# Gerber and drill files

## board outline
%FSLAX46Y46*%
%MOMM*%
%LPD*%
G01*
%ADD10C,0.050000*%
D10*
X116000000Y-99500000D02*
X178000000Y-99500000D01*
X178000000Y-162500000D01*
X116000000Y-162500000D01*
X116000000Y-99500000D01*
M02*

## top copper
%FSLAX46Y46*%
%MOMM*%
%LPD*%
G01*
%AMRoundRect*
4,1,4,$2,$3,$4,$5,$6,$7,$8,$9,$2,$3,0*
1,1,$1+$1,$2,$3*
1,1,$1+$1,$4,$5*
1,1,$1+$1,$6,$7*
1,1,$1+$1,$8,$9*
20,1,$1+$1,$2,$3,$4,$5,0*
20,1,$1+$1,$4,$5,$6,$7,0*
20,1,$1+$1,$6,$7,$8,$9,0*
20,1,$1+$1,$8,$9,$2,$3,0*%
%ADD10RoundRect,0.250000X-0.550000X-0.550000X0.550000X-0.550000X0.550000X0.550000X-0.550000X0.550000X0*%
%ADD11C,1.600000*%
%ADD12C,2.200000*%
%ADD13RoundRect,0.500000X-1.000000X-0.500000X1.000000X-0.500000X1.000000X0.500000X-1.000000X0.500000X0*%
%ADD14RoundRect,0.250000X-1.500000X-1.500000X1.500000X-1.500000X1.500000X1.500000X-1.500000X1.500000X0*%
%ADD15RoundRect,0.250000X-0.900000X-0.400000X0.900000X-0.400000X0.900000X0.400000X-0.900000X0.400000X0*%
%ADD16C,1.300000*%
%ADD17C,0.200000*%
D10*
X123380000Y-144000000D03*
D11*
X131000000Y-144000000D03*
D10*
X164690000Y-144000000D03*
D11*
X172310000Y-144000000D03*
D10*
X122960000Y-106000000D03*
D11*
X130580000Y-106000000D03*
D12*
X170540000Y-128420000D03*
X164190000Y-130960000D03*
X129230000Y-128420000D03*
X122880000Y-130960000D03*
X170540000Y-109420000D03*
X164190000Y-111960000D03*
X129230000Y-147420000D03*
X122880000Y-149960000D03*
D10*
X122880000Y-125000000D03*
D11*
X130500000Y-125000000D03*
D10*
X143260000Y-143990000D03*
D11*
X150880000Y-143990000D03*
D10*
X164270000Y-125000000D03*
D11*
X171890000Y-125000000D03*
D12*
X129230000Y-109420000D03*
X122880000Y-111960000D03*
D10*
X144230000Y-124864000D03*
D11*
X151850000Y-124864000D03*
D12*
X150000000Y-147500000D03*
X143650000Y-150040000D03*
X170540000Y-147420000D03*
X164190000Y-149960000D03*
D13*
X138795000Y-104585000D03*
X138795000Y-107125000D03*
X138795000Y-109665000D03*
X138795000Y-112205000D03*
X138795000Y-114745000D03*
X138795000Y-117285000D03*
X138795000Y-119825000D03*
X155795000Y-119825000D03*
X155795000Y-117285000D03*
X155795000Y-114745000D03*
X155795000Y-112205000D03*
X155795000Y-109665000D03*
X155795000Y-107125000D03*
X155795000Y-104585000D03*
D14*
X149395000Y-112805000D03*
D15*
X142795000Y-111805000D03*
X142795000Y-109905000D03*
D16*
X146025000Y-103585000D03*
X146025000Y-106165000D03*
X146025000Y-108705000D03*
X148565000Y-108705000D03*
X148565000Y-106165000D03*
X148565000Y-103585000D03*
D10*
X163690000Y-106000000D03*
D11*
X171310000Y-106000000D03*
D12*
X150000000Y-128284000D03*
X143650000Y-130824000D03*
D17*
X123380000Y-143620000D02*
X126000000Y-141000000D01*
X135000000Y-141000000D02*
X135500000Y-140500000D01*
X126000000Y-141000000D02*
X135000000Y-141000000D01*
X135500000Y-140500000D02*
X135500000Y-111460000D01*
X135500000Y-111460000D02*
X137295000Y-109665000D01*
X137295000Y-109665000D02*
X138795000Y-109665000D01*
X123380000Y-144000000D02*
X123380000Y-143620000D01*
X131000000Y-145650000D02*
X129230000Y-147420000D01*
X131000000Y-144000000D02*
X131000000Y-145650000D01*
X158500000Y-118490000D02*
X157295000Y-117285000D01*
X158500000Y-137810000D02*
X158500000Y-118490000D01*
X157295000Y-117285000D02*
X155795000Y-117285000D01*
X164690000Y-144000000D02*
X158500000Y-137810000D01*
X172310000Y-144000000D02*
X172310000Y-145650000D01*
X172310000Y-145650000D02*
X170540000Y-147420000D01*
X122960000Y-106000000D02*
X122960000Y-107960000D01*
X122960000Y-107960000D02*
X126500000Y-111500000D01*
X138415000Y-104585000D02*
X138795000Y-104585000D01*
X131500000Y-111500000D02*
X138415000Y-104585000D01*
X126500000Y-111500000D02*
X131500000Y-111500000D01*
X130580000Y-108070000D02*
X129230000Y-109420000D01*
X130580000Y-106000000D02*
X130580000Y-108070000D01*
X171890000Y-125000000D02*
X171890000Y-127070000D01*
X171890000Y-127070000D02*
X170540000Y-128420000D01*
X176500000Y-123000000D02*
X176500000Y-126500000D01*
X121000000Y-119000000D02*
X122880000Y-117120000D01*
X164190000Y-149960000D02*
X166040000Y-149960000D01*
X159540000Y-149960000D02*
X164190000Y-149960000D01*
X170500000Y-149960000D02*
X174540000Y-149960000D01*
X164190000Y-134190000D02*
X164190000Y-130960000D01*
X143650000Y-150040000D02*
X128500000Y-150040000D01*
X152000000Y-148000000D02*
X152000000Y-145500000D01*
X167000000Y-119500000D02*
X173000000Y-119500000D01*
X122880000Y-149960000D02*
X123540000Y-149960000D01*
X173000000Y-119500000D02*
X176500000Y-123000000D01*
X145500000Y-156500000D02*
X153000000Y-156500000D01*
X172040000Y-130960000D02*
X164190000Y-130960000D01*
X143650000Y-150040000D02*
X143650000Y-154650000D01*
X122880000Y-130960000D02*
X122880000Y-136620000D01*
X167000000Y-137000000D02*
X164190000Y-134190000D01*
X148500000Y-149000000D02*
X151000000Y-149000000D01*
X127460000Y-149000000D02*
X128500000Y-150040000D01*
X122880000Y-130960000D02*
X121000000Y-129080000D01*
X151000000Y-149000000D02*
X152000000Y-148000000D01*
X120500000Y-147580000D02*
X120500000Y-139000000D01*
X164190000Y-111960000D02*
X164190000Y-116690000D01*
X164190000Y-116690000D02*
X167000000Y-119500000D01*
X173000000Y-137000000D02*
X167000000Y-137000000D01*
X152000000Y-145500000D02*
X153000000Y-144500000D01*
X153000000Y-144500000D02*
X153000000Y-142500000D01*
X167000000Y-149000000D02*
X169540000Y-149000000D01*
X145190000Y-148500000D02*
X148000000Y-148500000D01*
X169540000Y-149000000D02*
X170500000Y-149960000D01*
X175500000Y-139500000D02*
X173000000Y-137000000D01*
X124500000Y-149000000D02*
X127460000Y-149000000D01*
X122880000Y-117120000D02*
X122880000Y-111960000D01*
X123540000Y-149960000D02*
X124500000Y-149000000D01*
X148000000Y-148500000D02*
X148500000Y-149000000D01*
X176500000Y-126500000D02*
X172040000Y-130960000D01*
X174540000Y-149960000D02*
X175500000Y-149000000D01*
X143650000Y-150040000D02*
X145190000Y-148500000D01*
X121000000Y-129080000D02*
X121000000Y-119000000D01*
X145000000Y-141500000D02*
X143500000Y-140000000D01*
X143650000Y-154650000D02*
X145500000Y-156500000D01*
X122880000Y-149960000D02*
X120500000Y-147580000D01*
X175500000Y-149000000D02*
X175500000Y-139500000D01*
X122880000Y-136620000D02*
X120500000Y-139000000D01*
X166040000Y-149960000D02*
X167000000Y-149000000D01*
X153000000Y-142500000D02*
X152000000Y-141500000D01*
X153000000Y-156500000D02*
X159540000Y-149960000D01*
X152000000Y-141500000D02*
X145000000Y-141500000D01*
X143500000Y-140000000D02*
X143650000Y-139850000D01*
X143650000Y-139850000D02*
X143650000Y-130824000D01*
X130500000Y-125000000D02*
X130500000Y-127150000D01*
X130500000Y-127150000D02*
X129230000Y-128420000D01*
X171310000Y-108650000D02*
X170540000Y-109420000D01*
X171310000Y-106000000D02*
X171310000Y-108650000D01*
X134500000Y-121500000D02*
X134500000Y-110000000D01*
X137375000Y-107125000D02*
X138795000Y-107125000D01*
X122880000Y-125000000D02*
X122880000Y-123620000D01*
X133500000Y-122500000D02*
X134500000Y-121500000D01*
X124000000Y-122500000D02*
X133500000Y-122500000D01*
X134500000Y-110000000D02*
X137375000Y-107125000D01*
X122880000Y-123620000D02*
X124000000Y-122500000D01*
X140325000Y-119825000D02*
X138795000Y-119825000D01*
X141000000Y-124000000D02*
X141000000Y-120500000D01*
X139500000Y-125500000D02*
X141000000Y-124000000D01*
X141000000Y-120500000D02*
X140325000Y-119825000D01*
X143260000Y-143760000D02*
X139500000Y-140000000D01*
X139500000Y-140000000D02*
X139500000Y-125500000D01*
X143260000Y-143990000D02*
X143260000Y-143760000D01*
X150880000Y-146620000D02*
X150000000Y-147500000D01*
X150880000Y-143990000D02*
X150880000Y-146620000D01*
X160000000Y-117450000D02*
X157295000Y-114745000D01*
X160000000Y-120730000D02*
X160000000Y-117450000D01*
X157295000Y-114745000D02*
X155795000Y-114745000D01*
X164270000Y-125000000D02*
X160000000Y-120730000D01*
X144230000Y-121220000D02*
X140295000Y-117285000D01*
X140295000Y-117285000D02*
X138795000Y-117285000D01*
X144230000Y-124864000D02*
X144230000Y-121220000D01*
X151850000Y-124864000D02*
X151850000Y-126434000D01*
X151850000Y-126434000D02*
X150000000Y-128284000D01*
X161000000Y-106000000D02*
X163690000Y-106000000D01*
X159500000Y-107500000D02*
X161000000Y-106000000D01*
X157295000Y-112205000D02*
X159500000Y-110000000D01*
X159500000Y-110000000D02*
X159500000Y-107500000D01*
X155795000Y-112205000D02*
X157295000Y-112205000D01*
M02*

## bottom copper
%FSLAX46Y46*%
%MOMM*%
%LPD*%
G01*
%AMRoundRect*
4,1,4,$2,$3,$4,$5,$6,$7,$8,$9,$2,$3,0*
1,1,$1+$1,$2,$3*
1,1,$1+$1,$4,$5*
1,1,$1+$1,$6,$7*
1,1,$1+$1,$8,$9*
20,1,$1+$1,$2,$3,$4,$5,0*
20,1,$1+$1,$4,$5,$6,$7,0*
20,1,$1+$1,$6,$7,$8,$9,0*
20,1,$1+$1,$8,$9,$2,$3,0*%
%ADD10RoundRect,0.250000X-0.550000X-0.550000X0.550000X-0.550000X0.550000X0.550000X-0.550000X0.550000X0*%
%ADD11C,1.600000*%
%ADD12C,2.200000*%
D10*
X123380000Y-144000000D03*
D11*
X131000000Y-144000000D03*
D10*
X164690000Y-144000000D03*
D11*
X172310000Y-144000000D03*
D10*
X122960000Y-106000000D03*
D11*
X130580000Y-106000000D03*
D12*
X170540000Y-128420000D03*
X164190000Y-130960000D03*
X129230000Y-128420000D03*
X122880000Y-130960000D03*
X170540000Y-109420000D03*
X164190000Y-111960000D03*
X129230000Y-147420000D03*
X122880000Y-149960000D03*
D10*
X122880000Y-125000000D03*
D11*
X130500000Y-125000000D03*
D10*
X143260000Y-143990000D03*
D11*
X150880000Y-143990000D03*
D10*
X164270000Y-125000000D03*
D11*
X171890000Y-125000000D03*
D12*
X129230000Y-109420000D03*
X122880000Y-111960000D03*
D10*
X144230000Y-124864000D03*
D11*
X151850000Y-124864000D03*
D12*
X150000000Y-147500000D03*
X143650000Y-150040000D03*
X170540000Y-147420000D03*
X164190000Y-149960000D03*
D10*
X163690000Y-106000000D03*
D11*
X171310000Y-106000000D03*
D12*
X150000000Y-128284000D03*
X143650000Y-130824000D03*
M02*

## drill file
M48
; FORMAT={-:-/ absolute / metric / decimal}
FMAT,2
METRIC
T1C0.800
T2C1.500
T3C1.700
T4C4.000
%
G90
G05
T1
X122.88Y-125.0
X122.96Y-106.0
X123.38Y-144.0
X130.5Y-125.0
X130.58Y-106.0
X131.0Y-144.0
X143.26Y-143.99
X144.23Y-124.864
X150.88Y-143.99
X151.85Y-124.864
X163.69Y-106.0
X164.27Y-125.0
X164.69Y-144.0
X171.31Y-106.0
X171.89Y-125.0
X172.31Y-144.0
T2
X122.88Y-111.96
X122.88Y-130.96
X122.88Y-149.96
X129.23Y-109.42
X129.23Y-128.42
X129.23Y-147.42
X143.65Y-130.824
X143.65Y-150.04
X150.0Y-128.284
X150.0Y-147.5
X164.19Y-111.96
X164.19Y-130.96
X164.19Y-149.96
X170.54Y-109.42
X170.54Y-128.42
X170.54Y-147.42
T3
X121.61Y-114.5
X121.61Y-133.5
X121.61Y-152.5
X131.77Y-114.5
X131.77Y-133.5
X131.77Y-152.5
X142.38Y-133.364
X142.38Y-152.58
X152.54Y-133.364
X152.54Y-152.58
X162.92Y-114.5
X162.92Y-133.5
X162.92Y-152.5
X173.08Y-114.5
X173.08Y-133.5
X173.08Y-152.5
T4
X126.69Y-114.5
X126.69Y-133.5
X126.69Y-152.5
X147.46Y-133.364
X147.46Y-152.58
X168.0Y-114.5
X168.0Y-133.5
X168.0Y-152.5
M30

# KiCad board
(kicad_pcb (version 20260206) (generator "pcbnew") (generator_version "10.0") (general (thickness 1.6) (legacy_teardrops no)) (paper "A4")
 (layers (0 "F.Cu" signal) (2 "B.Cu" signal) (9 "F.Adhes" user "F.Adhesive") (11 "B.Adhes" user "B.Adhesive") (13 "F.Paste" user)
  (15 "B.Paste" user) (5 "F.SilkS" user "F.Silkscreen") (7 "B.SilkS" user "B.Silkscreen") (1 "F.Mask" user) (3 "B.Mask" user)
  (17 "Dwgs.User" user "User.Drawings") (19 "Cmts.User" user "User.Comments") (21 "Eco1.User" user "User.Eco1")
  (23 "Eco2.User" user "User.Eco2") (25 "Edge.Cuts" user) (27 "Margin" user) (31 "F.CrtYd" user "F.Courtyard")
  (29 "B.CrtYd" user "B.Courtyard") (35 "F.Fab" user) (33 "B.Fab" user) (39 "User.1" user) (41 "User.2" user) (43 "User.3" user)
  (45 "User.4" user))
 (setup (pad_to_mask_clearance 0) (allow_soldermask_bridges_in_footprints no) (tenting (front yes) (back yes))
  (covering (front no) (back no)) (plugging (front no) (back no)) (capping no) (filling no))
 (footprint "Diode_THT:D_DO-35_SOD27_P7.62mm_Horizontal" (layer "F.Cu") (at 123.38 144)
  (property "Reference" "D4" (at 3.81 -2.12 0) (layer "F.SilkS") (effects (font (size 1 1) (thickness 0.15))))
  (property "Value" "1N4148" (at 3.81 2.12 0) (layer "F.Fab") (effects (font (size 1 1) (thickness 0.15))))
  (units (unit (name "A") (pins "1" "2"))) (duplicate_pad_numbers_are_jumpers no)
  (pad "1" thru_hole roundrect (at 0 0) (size 1.6 1.6) (drill 0.8) (layers "*.Cu" "*.Mask") (remove_unused_layers no)
   (roundrect_rratio 0.15625) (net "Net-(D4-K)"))
  (pad "2" thru_hole circle (at 7.62 0) (size 1.6 1.6) (drill 0.8) (layers "*.Cu" "*.Mask") (remove_unused_layers no) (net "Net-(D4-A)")))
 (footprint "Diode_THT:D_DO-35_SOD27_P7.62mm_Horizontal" (layer "F.Cu") (at 164.69 144)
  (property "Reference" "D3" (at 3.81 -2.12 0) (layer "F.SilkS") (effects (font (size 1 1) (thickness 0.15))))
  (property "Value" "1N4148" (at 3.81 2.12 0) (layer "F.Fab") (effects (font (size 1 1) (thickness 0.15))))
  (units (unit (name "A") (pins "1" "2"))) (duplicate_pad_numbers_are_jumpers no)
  (pad "1" thru_hole roundrect (at 0 0) (size 1.6 1.6) (drill 0.8) (layers "*.Cu" "*.Mask") (remove_unused_layers no)
   (roundrect_rratio 0.15625) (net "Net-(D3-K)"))
  (pad "2" thru_hole circle (at 7.62 0) (size 1.6 1.6) (drill 0.8) (layers "*.Cu" "*.Mask") (remove_unused_layers no) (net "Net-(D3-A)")))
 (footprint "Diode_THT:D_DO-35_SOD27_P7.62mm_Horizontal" (layer "F.Cu") (at 122.96 106)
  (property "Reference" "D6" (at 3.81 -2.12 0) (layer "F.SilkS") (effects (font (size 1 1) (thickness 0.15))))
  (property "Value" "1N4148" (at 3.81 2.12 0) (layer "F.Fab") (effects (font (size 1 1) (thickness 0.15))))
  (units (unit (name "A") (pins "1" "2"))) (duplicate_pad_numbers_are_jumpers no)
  (pad "1" thru_hole roundrect (at 0 0) (size 1.6 1.6) (drill 0.8) (layers "*.Cu" "*.Mask") (remove_unused_layers no)
   (roundrect_rratio 0.15625) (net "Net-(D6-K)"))
  (pad "2" thru_hole circle (at 7.62 0) (size 1.6 1.6) (drill 0.8) (layers "*.Cu" "*.Mask") (remove_unused_layers no) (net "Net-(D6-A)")))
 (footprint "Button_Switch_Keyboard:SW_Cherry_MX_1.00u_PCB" (layer "F.Cu") (at 170.54 128.42)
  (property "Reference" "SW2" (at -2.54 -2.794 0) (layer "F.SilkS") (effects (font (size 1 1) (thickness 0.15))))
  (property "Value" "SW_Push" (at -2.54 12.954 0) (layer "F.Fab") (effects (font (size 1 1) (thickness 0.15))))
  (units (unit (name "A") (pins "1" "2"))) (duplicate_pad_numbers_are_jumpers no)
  (pad "" np_thru_hole circle (at -7.62 5.08) (size 1.7 1.7) (drill 1.7) (layers "*.Cu" "*.Mask"))
  (pad "" np_thru_hole circle (at -2.54 5.08) (size 4 4) (drill 4) (layers "*.Cu" "*.Mask"))
  (pad "" np_thru_hole circle (at 2.54 5.08) (size 1.7 1.7) (drill 1.7) (layers "*.Cu" "*.Mask"))
  (pad "1" thru_hole circle (at 0 0) (size 2.2 2.2) (drill 1.5) (layers "*.Cu" "*.Mask") (remove_unused_layers no) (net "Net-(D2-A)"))
  (pad "2" thru_hole circle (at -6.35 2.54) (size 2.2 2.2) (drill 1.5) (layers "*.Cu" "*.Mask") (remove_unused_layers no) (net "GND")))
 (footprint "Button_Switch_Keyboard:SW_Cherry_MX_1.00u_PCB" (layer "F.Cu") (at 129.23 128.42)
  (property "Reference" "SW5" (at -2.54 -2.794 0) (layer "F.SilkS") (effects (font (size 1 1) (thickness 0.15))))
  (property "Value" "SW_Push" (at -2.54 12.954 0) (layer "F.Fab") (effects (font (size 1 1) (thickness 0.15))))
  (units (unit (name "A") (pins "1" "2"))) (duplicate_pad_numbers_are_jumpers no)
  (pad "" np_thru_hole circle (at -7.62 5.08) (size 1.7 1.7) (drill 1.7) (layers "*.Cu" "*.Mask"))
  (pad "" np_thru_hole circle (at -2.54 5.08) (size 4 4) (drill 4) (layers "*.Cu" "*.Mask"))
  (pad "" np_thru_hole circle (at 2.54 5.08) (size 1.7 1.7) (drill 1.7) (layers "*.Cu" "*.Mask"))
  (pad "1" thru_hole circle (at 0 0) (size 2.2 2.2) (drill 1.5) (layers "*.Cu" "*.Mask") (remove_unused_layers no) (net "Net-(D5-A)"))
  (pad "2" thru_hole circle (at -6.35 2.54) (size 2.2 2.2) (drill 1.5) (layers "*.Cu" "*.Mask") (remove_unused_layers no) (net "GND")))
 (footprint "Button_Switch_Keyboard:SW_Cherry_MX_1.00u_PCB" (layer "F.Cu") (at 170.54 109.42)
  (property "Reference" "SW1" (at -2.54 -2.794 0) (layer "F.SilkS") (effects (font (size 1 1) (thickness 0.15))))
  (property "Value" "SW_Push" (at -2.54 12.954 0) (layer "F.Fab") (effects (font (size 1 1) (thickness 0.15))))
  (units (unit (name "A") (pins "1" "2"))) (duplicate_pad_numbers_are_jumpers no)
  (pad "" np_thru_hole circle (at -7.62 5.08) (size 1.7 1.7) (drill 1.7) (layers "*.Cu" "*.Mask"))
  (pad "" np_thru_hole circle (at -2.54 5.08) (size 4 4) (drill 4) (layers "*.Cu" "*.Mask"))
  (pad "" np_thru_hole circle (at 2.54 5.08) (size 1.7 1.7) (drill 1.7) (layers "*.Cu" "*.Mask"))
  (pad "1" thru_hole circle (at 0 0) (size 2.2 2.2) (drill 1.5) (layers "*.Cu" "*.Mask") (remove_unused_layers no) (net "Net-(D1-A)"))
  (pad "2" thru_hole circle (at -6.35 2.54) (size 2.2 2.2) (drill 1.5) (layers "*.Cu" "*.Mask") (remove_unused_layers no) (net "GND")))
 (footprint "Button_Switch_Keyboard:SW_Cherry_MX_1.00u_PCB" (layer "F.Cu") (at 129.23 147.42)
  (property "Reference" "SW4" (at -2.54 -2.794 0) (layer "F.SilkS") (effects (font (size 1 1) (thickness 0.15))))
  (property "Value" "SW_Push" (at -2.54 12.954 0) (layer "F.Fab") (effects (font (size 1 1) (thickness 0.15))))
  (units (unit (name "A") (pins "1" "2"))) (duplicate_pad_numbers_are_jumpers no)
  (pad "" np_thru_hole circle (at -7.62 5.08) (size 1.7 1.7) (drill 1.7) (layers "*.Cu" "*.Mask"))
  (pad "" np_thru_hole circle (at -2.54 5.08) (size 4 4) (drill 4) (layers "*.Cu" "*.Mask"))
  (pad "" np_thru_hole circle (at 2.54 5.08) (size 1.7 1.7) (drill 1.7) (layers "*.Cu" "*.Mask"))
  (pad "1" thru_hole circle (at 0 0) (size 2.2 2.2) (drill 1.5) (layers "*.Cu" "*.Mask") (remove_unused_layers no) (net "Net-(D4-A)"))
  (pad "2" thru_hole circle (at -6.35 2.54) (size 2.2 2.2) (drill 1.5) (layers "*.Cu" "*.Mask") (remove_unused_layers no) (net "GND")))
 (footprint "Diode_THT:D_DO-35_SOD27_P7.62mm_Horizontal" (layer "F.Cu") (at 122.88 125)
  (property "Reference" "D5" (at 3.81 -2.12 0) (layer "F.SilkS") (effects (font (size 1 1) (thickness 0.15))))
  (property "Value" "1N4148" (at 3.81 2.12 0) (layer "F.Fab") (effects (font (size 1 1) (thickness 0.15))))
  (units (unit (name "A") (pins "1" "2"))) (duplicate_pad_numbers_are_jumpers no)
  (pad "1" thru_hole roundrect (at 0 0) (size 1.6 1.6) (drill 0.8) (layers "*.Cu" "*.Mask") (remove_unused_layers no)
   (roundrect_rratio 0.15625) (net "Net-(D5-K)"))
  (pad "2" thru_hole circle (at 7.62 0) (size 1.6 1.6) (drill 0.8) (layers "*.Cu" "*.Mask") (remove_unused_layers no) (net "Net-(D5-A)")))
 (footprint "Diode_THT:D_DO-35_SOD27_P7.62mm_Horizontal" (layer "F.Cu") (at 143.26 143.99)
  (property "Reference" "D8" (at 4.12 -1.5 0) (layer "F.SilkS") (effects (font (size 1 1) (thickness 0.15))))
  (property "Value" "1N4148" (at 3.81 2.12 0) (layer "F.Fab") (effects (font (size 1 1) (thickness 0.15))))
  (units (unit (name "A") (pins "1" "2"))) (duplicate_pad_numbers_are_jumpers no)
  (pad "1" thru_hole roundrect (at 0 0) (size 1.6 1.6) (drill 0.8) (layers "*.Cu" "*.Mask") (remove_unused_layers no)
   (roundrect_rratio 0.15625) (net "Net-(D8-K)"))
  (pad "2" thru_hole circle (at 7.62 0) (size 1.6 1.6) (drill 0.8) (layers "*.Cu" "*.Mask") (remove_unused_layers no) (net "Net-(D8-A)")))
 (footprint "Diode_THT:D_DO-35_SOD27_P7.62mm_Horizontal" (layer "F.Cu") (at 164.27 125)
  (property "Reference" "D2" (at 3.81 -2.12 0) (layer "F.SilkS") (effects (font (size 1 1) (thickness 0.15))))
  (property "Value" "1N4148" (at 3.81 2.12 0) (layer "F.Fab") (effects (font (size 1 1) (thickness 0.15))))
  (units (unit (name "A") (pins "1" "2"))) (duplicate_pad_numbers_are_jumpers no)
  (pad "1" thru_hole roundrect (at 0 0) (size 1.6 1.6) (drill 0.8) (layers "*.Cu" "*.Mask") (remove_unused_layers no)
   (roundrect_rratio 0.15625) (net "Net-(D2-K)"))
  (pad "2" thru_hole circle (at 7.62 0) (size 1.6 1.6) (drill 0.8) (layers "*.Cu" "*.Mask") (remove_unused_layers no) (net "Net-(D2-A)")))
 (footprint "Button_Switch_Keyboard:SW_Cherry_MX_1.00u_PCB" (layer "F.Cu") (at 129.23 109.42)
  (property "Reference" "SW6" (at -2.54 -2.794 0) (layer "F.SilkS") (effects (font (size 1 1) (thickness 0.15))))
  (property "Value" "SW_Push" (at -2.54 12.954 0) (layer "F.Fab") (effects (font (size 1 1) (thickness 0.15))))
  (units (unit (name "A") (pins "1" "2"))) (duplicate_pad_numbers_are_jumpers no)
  (pad "" np_thru_hole circle (at -7.62 5.08) (size 1.7 1.7) (drill 1.7) (layers "*.Cu" "*.Mask"))
  (pad "" np_thru_hole circle (at -2.54 5.08) (size 4 4) (drill 4) (layers "*.Cu" "*.Mask"))
  (pad "" np_thru_hole circle (at 2.54 5.08) (size 1.7 1.7) (drill 1.7) (layers "*.Cu" "*.Mask"))
  (pad "1" thru_hole circle (at 0 0) (size 2.2 2.2) (drill 1.5) (layers "*.Cu" "*.Mask") (remove_unused_layers no) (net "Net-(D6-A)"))
  (pad "2" thru_hole circle (at -6.35 2.54) (size 2.2 2.2) (drill 1.5) (layers "*.Cu" "*.Mask") (remove_unused_layers no) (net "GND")))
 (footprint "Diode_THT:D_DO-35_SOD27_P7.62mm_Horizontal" (layer "F.Cu") (at 144.23 124.864)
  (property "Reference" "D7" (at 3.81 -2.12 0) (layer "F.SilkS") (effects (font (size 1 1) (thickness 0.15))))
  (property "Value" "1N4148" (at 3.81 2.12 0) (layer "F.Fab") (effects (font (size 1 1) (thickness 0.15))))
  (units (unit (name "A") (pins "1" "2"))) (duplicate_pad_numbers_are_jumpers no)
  (pad "1" thru_hole roundrect (at 0 0) (size 1.6 1.6) (drill 0.8) (layers "*.Cu" "*.Mask") (remove_unused_layers no)
   (roundrect_rratio 0.15625) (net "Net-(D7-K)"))
  (pad "2" thru_hole circle (at 7.62 0) (size 1.6 1.6) (drill 0.8) (layers "*.Cu" "*.Mask") (remove_unused_layers no) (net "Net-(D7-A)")))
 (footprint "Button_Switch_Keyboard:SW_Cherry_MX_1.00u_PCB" (layer "F.Cu") (at 150 147.5)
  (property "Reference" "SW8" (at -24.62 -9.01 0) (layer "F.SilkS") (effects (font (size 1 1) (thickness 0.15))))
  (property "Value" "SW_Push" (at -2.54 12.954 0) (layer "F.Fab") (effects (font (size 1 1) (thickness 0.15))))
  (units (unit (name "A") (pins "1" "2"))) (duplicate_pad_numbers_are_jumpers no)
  (pad "" np_thru_hole circle (at -7.62 5.08) (size 1.7 1.7) (drill 1.7) (layers "*.Cu" "*.Mask"))
  (pad "" np_thru_hole circle (at -2.54 5.08) (size 4 4) (drill 4) (layers "*.Cu" "*.Mask"))
  (pad "" np_thru_hole circle (at 2.54 5.08) (size 1.7 1.7) (drill 1.7) (layers "*.Cu" "*.Mask"))
  (pad "1" thru_hole circle (at 0 0) (size 2.2 2.2) (drill 1.5) (layers "*.Cu" "*.Mask") (remove_unused_layers no) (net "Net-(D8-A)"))
  (pad "2" thru_hole circle (at -6.35 2.54) (size 2.2 2.2) (drill 1.5) (layers "*.Cu" "*.Mask") (remove_unused_layers no) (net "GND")))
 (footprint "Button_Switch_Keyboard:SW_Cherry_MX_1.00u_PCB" (layer "F.Cu") (at 170.54 147.42)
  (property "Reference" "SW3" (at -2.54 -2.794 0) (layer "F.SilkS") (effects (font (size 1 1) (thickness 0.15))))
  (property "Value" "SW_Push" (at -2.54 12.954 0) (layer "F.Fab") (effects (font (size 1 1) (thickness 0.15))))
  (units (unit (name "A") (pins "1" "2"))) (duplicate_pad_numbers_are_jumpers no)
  (pad "" np_thru_hole circle (at -7.62 5.08) (size 1.7 1.7) (drill 1.7) (layers "*.Cu" "*.Mask"))
  (pad "" np_thru_hole circle (at -2.54 5.08) (size 4 4) (drill 4) (layers "*.Cu" "*.Mask"))
  (pad "" np_thru_hole circle (at 2.54 5.08) (size 1.7 1.7) (drill 1.7) (layers "*.Cu" "*.Mask"))
  (pad "1" thru_hole circle (at 0 0) (size 2.2 2.2) (drill 1.5) (layers "*.Cu" "*.Mask") (remove_unused_layers no) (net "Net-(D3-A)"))
  (pad "2" thru_hole circle (at -6.35 2.54) (size 2.2 2.2) (drill 1.5) (layers "*.Cu" "*.Mask") (remove_unused_layers no) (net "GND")))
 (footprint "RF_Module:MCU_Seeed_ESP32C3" (layer "F.Cu") (at 147.295 112.205)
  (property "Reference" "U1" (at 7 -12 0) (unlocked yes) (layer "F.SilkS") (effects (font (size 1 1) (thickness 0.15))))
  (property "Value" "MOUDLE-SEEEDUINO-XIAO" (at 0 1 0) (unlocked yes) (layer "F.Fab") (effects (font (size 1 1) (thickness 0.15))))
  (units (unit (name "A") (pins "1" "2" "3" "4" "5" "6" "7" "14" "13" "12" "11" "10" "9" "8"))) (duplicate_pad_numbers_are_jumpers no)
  (pad "" smd roundrect (at 1.1 -0.4) (size 1.5 1.5) (layers "F.Paste") (roundrect_rratio 0.1666666667))
  (pad "" smd roundrect (at 1.1 1.6) (size 1.5 1.5) (layers "F.Paste") (roundrect_rratio 0.1666666667))
  (pad "" smd roundrect (at 3.1 -0.4) (size 1.5 1.5) (layers "F.Paste") (roundrect_rratio 0.1666666667))
  (pad "" smd roundrect (at 3.1 1.6) (size 1.5 1.5) (layers "F.Paste") (roundrect_rratio 0.1666666667))
  (pad "1" smd roundrect (at -8.5 -7.62) (size 3 2) (layers "F.Cu" "F.Mask" "F.Paste") (roundrect_rratio 0.25) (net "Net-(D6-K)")
   (thermal_bridge_angle 45))
  (pad "2" smd roundrect (at -8.5 -5.08) (size 3 2) (layers "F.Cu" "F.Mask" "F.Paste") (roundrect_rratio 0.25) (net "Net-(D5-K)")
   (thermal_bridge_angle 45))
  (pad "3" smd roundrect (at -8.5 -2.54) (size 3 2) (layers "F.Cu" "F.Mask" "F.Paste") (roundrect_rratio 0.25) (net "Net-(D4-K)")
   (thermal_bridge_angle 45))
  (pad "4" smd roundrect (at -8.5 0) (size 3 2) (layers "F.Cu" "F.Mask" "F.Paste") (roundrect_rratio 0.25)
   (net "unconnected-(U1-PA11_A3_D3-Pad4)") (thermal_bridge_angle 45))
  (pad "5" smd roundrect (at -8.5 2.54) (size 3 2) (layers "F.Cu" "F.Mask" "F.Paste") (roundrect_rratio 0.25)
   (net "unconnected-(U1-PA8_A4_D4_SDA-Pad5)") (thermal_bridge_angle 45))
  (pad "6" smd roundrect (at -8.5 5.08) (size 3 2) (layers "F.Cu" "F.Mask" "F.Paste") (roundrect_rratio 0.25) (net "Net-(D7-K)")
   (thermal_bridge_angle 45))
  (pad "7" smd roundrect (at -8.5 7.62) (size 3 2) (layers "F.Cu" "F.Mask" "F.Paste") (roundrect_rratio 0.25) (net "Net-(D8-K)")
   (thermal_bridge_angle 45))
  (pad "8" smd roundrect (at 8.5 7.62) (size 3 2) (layers "F.Cu" "F.Mask" "F.Paste") (roundrect_rratio 0.25)
   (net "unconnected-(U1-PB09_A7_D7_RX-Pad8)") (thermal_bridge_angle 45))
  (pad "9" smd roundrect (at 8.5 5.08) (size 3 2) (layers "F.Cu" "F.Mask" "F.Paste") (roundrect_rratio 0.25) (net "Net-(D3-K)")
   (thermal_bridge_angle 45))
  (pad "10" smd roundrect (at 8.5 2.54) (size 3 2) (layers "F.Cu" "F.Mask" "F.Paste") (roundrect_rratio 0.25) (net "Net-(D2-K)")
   (thermal_bridge_angle 45))
  (pad "11" smd roundrect (at 8.5 0) (size 3 2) (layers "F.Cu" "F.Mask" "F.Paste") (roundrect_rratio 0.25) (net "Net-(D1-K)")
   (thermal_bridge_angle 45))
  (pad "12" smd roundrect (at 8.5 -2.54) (size 3 2) (layers "F.Cu" "F.Mask" "F.Paste") (roundrect_rratio 0.25)
   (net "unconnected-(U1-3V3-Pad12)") (thermal_bridge_angle 45))
  (pad "13" smd roundrect (at 8.5 -5.08) (size 3 2) (layers "F.Cu" "F.Mask" "F.Paste") (roundrect_rratio 0.25)
   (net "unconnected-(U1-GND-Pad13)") (thermal_bridge_angle 45))
  (pad "14" smd roundrect (at 8.5 -7.62) (size 3 2) (layers "F.Cu" "F.Mask" "F.Paste") (roundrect_rratio 0.25)
   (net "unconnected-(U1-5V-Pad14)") (thermal_bridge_angle 45))
  (pad "15" smd roundrect (at 2.1 0.6) (size 3.5 3.5) (layers "F.Cu" "F.Mask") (roundrect_rratio 0.07142857143))
  (pad "16" smd roundrect (at -4.5 -0.4) (size 2.3 1.3) (layers "F.Cu" "F.Mask" "F.Paste") (roundrect_rratio 0.1923076923))
  (pad "17" smd roundrect (at -4.5 -2.3) (size 2.3 1.3) (layers "F.Cu" "F.Mask" "F.Paste") (roundrect_rratio 0.1923076923))
  (pad "18" smd circle (at -1.27 -8.62) (size 1.3 1.3) (layers "F.Cu" "F.Mask" "F.Paste"))
  (pad "19" smd circle (at -1.27 -6.04) (size 1.3 1.3) (layers "F.Cu" "F.Mask" "F.Paste"))
  (pad "20" smd circle (at -1.27 -3.5) (size 1.3 1.3) (layers "F.Cu" "F.Mask" "F.Paste"))
  (pad "21" smd circle (at 1.27 -3.5) (size 1.3 1.3) (layers "F.Cu" "F.Mask" "F.Paste"))
  (pad "22" smd circle (at 1.27 -6.04) (size 1.3 1.3) (layers "F.Cu" "F.Mask" "F.Paste"))
  (pad "23" smd circle (at 1.27 -8.62) (size 1.3 1.3) (layers "F.Cu" "F.Mask" "F.Paste")))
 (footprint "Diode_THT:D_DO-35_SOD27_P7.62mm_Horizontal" (layer "F.Cu") (at 163.69 106)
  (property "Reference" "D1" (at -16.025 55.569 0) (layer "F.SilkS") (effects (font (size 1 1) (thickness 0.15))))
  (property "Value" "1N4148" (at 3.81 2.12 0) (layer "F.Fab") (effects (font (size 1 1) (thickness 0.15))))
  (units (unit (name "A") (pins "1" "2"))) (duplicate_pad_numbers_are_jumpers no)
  (pad "1" thru_hole roundrect (at 0 0) (size 1.6 1.6) (drill 0.8) (layers "*.Cu" "*.Mask") (remove_unused_layers no)
   (roundrect_rratio 0.15625) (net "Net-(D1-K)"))
  (pad "2" thru_hole circle (at 7.62 0) (size 1.6 1.6) (drill 0.8) (layers "*.Cu" "*.Mask") (remove_unused_layers no) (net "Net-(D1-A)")))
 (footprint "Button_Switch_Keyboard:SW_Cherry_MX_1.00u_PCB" (layer "F.Cu") (at 150 128.284)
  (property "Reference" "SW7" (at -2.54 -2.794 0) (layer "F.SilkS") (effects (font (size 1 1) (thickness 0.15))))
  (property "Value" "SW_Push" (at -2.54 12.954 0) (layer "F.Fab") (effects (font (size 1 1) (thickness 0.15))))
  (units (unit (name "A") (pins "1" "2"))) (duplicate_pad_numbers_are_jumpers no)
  (pad "" np_thru_hole circle (at -7.62 5.08) (size 1.7 1.7) (drill 1.7) (layers "*.Cu" "*.Mask"))
  (pad "" np_thru_hole circle (at -2.54 5.08) (size 4 4) (drill 4) (layers "*.Cu" "*.Mask"))
  (pad "" np_thru_hole circle (at 2.54 5.08) (size 1.7 1.7) (drill 1.7) (layers "*.Cu" "*.Mask"))
  (pad "1" thru_hole circle (at 0 0) (size 2.2 2.2) (drill 1.5) (layers "*.Cu" "*.Mask") (remove_unused_layers no) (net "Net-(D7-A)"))
  (pad "2" thru_hole circle (at -6.35 2.54) (size 2.2 2.2) (drill 1.5) (layers "*.Cu" "*.Mask") (remove_unused_layers no) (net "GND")))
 (gr_rect (start 116 99.5) (end 178 162.5) (stroke (width 0.05) (type default)) (fill no) (layer "Edge.Cuts"))
 (segment (start 123.38 143.62) (end 126 141) (width 0.2) (layer "F.Cu") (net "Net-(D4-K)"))
 (segment (start 135 141) (end 135.5 140.5) (width 0.2) (layer "F.Cu") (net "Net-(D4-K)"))
 (segment (start 126 141) (end 135 141) (width 0.2) (layer "F.Cu") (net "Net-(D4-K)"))
 (segment (start 135.5 140.5) (end 135.5 111.46) (width 0.2) (layer "F.Cu") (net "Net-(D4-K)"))
 (segment (start 135.5 111.46) (end 137.295 109.665) (width 0.2) (layer "F.Cu") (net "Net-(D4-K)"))
 (segment (start 137.295 109.665) (end 138.795 109.665) (width 0.2) (layer "F.Cu") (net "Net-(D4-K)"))
 (segment (start 123.38 144) (end 123.38 143.62) (width 0.2) (layer "F.Cu") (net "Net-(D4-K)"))
 (segment (start 131 145.65) (end 129.23 147.42) (width 0.2) (layer "F.Cu") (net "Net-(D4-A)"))
 (segment (start 131 144) (end 131 145.65) (width 0.2) (layer "F.Cu") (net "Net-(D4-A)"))
 (segment (start 158.5 118.49) (end 157.295 117.285) (width 0.2) (layer "F.Cu") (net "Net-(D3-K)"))
 (segment (start 158.5 137.81) (end 158.5 118.49) (width 0.2) (layer "F.Cu") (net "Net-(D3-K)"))
 (segment (start 157.295 117.285) (end 155.795 117.285) (width 0.2) (layer "F.Cu") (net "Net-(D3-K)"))
 (segment (start 164.69 144) (end 158.5 137.81) (width 0.2) (layer "F.Cu") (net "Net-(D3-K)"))
 (segment (start 172.31 144) (end 172.31 145.65) (width 0.2) (layer "F.Cu") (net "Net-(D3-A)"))
 (segment (start 172.31 145.65) (end 170.54 147.42) (width 0.2) (layer "F.Cu") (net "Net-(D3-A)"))
 (segment (start 122.96 106) (end 122.96 107.96) (width 0.2) (layer "F.Cu") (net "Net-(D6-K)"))
 (segment (start 122.96 107.96) (end 126.5 111.5) (width 0.2) (layer "F.Cu") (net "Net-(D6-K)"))
 (segment (start 138.415 104.585) (end 138.795 104.585) (width 0.2) (layer "F.Cu") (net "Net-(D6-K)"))
 (segment (start 131.5 111.5) (end 138.415 104.585) (width 0.2) (layer "F.Cu") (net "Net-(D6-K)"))
 (segment (start 126.5 111.5) (end 131.5 111.5) (width 0.2) (layer "F.Cu") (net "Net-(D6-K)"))
 (segment (start 130.58 108.07) (end 129.23 109.42) (width 0.2) (layer "F.Cu") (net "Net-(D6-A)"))
 (segment (start 130.58 106) (end 130.58 108.07) (width 0.2) (layer "F.Cu") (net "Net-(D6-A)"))
 (segment (start 171.89 125) (end 171.89 127.07) (width 0.2) (layer "F.Cu") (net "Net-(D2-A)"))
 (segment (start 171.89 127.07) (end 170.54 128.42) (width 0.2) (layer "F.Cu") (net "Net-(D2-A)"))
 (segment (start 176.5 123) (end 176.5 126.5) (width 0.2) (layer "F.Cu") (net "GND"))
 (segment (start 121 119) (end 122.88 117.12) (width 0.2) (layer "F.Cu") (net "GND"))
 (segment (start 164.19 149.96) (end 166.04 149.96) (width 0.2) (layer "F.Cu") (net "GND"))
 (segment (start 159.54 149.96) (end 164.19 149.96) (width 0.2) (layer "F.Cu") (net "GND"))
 (segment (start 170.5 149.96) (end 174.54 149.96) (width 0.2) (layer "F.Cu") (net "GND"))
 (segment (start 164.19 134.19) (end 164.19 130.96) (width 0.2) (layer "F.Cu") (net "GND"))
 (segment (start 143.65 150.04) (end 128.5 150.04) (width 0.2) (layer "F.Cu") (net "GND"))
 (segment (start 152 148) (end 152 145.5) (width 0.2) (layer "F.Cu") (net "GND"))
 (segment (start 167 119.5) (end 173 119.5) (width 0.2) (layer "F.Cu") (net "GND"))
 (segment (start 122.88 149.96) (end 123.54 149.96) (width 0.2) (layer "F.Cu") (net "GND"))
 (segment (start 173 119.5) (end 176.5 123) (width 0.2) (layer "F.Cu") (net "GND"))
 (segment (start 145.5 156.5) (end 153 156.5) (width 0.2) (layer "F.Cu") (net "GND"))
 (segment (start 172.04 130.96) (end 164.19 130.96) (width 0.2) (layer "F.Cu") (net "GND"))
 (segment (start 143.65 150.04) (end 143.65 154.65) (width 0.2) (layer "F.Cu") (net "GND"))
 (segment (start 122.88 130.96) (end 122.88 136.62) (width 0.2) (layer "F.Cu") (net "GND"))
 (segment (start 167 137) (end 164.19 134.19) (width 0.2) (layer "F.Cu") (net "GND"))
 (segment (start 148.5 149) (end 151 149) (width 0.2) (layer "F.Cu") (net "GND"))
 (segment (start 127.46 149) (end 128.5 150.04) (width 0.2) (layer "F.Cu") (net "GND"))
 (segment (start 122.88 130.96) (end 121 129.08) (width 0.2) (layer "F.Cu") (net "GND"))
 (segment (start 151 149) (end 152 148) (width 0.2) (layer "F.Cu") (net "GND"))
 (segment (start 120.5 147.58) (end 120.5 139) (width 0.2) (layer "F.Cu") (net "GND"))
 (segment (start 164.19 111.96) (end 164.19 116.69) (width 0.2) (layer "F.Cu") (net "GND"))
 (segment (start 164.19 116.69) (end 167 119.5) (width 0.2) (layer "F.Cu") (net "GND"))
 (segment (start 173 137) (end 167 137) (width 0.2) (layer "F.Cu") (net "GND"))
 (segment (start 152 145.5) (end 153 144.5) (width 0.2) (layer "F.Cu") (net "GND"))
 (segment (start 153 144.5) (end 153 142.5) (width 0.2) (layer "F.Cu") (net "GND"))
 (segment (start 167 149) (end 169.54 149) (width 0.2) (layer "F.Cu") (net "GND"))
 (segment (start 145.19 148.5) (end 148 148.5) (width 0.2) (layer "F.Cu") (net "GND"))
 (segment (start 169.54 149) (end 170.5 149.96) (width 0.2) (layer "F.Cu") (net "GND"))
 (segment (start 175.5 139.5) (end 173 137) (width 0.2) (layer "F.Cu") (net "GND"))
 (segment (start 124.5 149) (end 127.46 149) (width 0.2) (layer "F.Cu") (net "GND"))
 (segment (start 122.88 117.12) (end 122.88 111.96) (width 0.2) (layer "F.Cu") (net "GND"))
 (segment (start 123.54 149.96) (end 124.5 149) (width 0.2) (layer "F.Cu") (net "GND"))
 (segment (start 148 148.5) (end 148.5 149) (width 0.2) (layer "F.Cu") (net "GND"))
 (segment (start 176.5 126.5) (end 172.04 130.96) (width 0.2) (layer "F.Cu") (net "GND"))
 (segment (start 174.54 149.96) (end 175.5 149) (width 0.2) (layer "F.Cu") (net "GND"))
 (segment (start 143.65 150.04) (end 145.19 148.5) (width 0.2) (layer "F.Cu") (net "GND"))
 (segment (start 121 129.08) (end 121 119) (width 0.2) (layer "F.Cu") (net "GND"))
 (segment (start 145 141.5) (end 143.5 140) (width 0.2) (layer "F.Cu") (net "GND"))
 (segment (start 143.65 154.65) (end 145.5 156.5) (width 0.2) (layer "F.Cu") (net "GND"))
 (segment (start 122.88 149.96) (end 120.5 147.58) (width 0.2) (layer "F.Cu") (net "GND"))
 (segment (start 175.5 149) (end 175.5 139.5) (width 0.2) (layer "F.Cu") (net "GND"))
 (segment (start 122.88 136.62) (end 120.5 139) (width 0.2) (layer "F.Cu") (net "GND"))
 (segment (start 166.04 149.96) (end 167 149) (width 0.2) (layer "F.Cu") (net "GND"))
 (segment (start 153 142.5) (end 152 141.5) (width 0.2) (layer "F.Cu") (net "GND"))
 (segment (start 153 156.5) (end 159.54 149.96) (width 0.2) (layer "F.Cu") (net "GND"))
 (segment (start 152 141.5) (end 145 141.5) (width 0.2) (layer "F.Cu") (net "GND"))
 (segment (start 143.5 140) (end 143.65 139.85) (width 0.2) (layer "F.Cu") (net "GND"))
 (segment (start 143.65 139.85) (end 143.65 130.824) (width 0.2) (layer "F.Cu") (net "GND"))
 (segment (start 130.5 125) (end 130.5 127.15) (width 0.2) (layer "F.Cu") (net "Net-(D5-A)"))
 (segment (start 130.5 127.15) (end 129.23 128.42) (width 0.2) (layer "F.Cu") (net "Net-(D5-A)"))
 (segment (start 171.31 108.65) (end 170.54 109.42) (width 0.2) (layer "F.Cu") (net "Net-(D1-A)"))
 (segment (start 171.31 106) (end 171.31 108.65) (width 0.2) (layer "F.Cu") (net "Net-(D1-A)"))
 (segment (start 134.5 121.5) (end 134.5 110) (width 0.2) (layer "F.Cu") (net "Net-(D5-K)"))
 (segment (start 137.375 107.125) (end 138.795 107.125) (width 0.2) (layer "F.Cu") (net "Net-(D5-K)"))
 (segment (start 122.88 125) (end 122.88 123.62) (width 0.2) (layer "F.Cu") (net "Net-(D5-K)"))
 (segment (start 133.5 122.5) (end 134.5 121.5) (width 0.2) (layer "F.Cu") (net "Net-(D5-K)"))
 (segment (start 124 122.5) (end 133.5 122.5) (width 0.2) (layer "F.Cu") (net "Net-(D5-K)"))
 (segment (start 134.5 110) (end 137.375 107.125) (width 0.2) (layer "F.Cu") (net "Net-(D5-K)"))
 (segment (start 122.88 123.62) (end 124 122.5) (width 0.2) (layer "F.Cu") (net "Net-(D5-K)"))
 (segment (start 140.325 119.825) (end 138.795 119.825) (width 0.2) (layer "F.Cu") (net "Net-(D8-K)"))
 (segment (start 141 124) (end 141 120.5) (width 0.2) (layer "F.Cu") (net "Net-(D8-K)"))
 (segment (start 139.5 125.5) (end 141 124) (width 0.2) (layer "F.Cu") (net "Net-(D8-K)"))
 (segment (start 141 120.5) (end 140.325 119.825) (width 0.2) (layer "F.Cu") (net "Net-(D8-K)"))
 (segment (start 143.26 143.76) (end 139.5 140) (width 0.2) (layer "F.Cu") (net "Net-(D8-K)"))
 (segment (start 139.5 140) (end 139.5 125.5) (width 0.2) (layer "F.Cu") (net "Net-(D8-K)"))
 (segment (start 143.26 143.99) (end 143.26 143.76) (width 0.2) (layer "F.Cu") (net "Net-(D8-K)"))
 (segment (start 150.88 146.62) (end 150 147.5) (width 0.2) (layer "F.Cu") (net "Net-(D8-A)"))
 (segment (start 150.88 143.99) (end 150.88 146.62) (width 0.2) (layer "F.Cu") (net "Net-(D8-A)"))
 (segment (start 160 117.45) (end 157.295 114.745) (width 0.2) (layer "F.Cu") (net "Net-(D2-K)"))
 (segment (start 160 120.73) (end 160 117.45) (width 0.2) (layer "F.Cu") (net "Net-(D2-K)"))
 (segment (start 157.295 114.745) (end 155.795 114.745) (width 0.2) (layer "F.Cu") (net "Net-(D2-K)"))
 (segment (start 164.27 125) (end 160 120.73) (width 0.2) (layer "F.Cu") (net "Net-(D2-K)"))
 (segment (start 144.23 121.22) (end 140.295 117.285) (width 0.2) (layer "F.Cu") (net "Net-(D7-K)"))
 (segment (start 140.295 117.285) (end 138.795 117.285) (width 0.2) (layer "F.Cu") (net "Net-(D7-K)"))
 (segment (start 144.23 124.864) (end 144.23 121.22) (width 0.2) (layer "F.Cu") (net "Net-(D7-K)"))
 (segment (start 151.85 124.864) (end 151.85 126.434) (width 0.2) (layer "F.Cu") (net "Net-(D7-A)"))
 (segment (start 151.85 126.434) (end 150 128.284) (width 0.2) (layer "F.Cu") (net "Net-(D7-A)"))
 (segment (start 161 106) (end 163.69 106) (width 0.2) (layer "F.Cu") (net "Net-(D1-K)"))
 (segment (start 159.5 107.5) (end 161 106) (width 0.2) (layer "F.Cu") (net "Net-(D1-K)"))
 (segment (start 157.295 112.205) (end 159.5 110) (width 0.2) (layer "F.Cu") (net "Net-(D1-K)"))
 (segment (start 159.5 110) (end 159.5 107.5) (width 0.2) (layer "F.Cu") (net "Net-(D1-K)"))
 (segment (start 155.795 112.205) (end 157.295 112.205) (width 0.2) (layer "F.Cu") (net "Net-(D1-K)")))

